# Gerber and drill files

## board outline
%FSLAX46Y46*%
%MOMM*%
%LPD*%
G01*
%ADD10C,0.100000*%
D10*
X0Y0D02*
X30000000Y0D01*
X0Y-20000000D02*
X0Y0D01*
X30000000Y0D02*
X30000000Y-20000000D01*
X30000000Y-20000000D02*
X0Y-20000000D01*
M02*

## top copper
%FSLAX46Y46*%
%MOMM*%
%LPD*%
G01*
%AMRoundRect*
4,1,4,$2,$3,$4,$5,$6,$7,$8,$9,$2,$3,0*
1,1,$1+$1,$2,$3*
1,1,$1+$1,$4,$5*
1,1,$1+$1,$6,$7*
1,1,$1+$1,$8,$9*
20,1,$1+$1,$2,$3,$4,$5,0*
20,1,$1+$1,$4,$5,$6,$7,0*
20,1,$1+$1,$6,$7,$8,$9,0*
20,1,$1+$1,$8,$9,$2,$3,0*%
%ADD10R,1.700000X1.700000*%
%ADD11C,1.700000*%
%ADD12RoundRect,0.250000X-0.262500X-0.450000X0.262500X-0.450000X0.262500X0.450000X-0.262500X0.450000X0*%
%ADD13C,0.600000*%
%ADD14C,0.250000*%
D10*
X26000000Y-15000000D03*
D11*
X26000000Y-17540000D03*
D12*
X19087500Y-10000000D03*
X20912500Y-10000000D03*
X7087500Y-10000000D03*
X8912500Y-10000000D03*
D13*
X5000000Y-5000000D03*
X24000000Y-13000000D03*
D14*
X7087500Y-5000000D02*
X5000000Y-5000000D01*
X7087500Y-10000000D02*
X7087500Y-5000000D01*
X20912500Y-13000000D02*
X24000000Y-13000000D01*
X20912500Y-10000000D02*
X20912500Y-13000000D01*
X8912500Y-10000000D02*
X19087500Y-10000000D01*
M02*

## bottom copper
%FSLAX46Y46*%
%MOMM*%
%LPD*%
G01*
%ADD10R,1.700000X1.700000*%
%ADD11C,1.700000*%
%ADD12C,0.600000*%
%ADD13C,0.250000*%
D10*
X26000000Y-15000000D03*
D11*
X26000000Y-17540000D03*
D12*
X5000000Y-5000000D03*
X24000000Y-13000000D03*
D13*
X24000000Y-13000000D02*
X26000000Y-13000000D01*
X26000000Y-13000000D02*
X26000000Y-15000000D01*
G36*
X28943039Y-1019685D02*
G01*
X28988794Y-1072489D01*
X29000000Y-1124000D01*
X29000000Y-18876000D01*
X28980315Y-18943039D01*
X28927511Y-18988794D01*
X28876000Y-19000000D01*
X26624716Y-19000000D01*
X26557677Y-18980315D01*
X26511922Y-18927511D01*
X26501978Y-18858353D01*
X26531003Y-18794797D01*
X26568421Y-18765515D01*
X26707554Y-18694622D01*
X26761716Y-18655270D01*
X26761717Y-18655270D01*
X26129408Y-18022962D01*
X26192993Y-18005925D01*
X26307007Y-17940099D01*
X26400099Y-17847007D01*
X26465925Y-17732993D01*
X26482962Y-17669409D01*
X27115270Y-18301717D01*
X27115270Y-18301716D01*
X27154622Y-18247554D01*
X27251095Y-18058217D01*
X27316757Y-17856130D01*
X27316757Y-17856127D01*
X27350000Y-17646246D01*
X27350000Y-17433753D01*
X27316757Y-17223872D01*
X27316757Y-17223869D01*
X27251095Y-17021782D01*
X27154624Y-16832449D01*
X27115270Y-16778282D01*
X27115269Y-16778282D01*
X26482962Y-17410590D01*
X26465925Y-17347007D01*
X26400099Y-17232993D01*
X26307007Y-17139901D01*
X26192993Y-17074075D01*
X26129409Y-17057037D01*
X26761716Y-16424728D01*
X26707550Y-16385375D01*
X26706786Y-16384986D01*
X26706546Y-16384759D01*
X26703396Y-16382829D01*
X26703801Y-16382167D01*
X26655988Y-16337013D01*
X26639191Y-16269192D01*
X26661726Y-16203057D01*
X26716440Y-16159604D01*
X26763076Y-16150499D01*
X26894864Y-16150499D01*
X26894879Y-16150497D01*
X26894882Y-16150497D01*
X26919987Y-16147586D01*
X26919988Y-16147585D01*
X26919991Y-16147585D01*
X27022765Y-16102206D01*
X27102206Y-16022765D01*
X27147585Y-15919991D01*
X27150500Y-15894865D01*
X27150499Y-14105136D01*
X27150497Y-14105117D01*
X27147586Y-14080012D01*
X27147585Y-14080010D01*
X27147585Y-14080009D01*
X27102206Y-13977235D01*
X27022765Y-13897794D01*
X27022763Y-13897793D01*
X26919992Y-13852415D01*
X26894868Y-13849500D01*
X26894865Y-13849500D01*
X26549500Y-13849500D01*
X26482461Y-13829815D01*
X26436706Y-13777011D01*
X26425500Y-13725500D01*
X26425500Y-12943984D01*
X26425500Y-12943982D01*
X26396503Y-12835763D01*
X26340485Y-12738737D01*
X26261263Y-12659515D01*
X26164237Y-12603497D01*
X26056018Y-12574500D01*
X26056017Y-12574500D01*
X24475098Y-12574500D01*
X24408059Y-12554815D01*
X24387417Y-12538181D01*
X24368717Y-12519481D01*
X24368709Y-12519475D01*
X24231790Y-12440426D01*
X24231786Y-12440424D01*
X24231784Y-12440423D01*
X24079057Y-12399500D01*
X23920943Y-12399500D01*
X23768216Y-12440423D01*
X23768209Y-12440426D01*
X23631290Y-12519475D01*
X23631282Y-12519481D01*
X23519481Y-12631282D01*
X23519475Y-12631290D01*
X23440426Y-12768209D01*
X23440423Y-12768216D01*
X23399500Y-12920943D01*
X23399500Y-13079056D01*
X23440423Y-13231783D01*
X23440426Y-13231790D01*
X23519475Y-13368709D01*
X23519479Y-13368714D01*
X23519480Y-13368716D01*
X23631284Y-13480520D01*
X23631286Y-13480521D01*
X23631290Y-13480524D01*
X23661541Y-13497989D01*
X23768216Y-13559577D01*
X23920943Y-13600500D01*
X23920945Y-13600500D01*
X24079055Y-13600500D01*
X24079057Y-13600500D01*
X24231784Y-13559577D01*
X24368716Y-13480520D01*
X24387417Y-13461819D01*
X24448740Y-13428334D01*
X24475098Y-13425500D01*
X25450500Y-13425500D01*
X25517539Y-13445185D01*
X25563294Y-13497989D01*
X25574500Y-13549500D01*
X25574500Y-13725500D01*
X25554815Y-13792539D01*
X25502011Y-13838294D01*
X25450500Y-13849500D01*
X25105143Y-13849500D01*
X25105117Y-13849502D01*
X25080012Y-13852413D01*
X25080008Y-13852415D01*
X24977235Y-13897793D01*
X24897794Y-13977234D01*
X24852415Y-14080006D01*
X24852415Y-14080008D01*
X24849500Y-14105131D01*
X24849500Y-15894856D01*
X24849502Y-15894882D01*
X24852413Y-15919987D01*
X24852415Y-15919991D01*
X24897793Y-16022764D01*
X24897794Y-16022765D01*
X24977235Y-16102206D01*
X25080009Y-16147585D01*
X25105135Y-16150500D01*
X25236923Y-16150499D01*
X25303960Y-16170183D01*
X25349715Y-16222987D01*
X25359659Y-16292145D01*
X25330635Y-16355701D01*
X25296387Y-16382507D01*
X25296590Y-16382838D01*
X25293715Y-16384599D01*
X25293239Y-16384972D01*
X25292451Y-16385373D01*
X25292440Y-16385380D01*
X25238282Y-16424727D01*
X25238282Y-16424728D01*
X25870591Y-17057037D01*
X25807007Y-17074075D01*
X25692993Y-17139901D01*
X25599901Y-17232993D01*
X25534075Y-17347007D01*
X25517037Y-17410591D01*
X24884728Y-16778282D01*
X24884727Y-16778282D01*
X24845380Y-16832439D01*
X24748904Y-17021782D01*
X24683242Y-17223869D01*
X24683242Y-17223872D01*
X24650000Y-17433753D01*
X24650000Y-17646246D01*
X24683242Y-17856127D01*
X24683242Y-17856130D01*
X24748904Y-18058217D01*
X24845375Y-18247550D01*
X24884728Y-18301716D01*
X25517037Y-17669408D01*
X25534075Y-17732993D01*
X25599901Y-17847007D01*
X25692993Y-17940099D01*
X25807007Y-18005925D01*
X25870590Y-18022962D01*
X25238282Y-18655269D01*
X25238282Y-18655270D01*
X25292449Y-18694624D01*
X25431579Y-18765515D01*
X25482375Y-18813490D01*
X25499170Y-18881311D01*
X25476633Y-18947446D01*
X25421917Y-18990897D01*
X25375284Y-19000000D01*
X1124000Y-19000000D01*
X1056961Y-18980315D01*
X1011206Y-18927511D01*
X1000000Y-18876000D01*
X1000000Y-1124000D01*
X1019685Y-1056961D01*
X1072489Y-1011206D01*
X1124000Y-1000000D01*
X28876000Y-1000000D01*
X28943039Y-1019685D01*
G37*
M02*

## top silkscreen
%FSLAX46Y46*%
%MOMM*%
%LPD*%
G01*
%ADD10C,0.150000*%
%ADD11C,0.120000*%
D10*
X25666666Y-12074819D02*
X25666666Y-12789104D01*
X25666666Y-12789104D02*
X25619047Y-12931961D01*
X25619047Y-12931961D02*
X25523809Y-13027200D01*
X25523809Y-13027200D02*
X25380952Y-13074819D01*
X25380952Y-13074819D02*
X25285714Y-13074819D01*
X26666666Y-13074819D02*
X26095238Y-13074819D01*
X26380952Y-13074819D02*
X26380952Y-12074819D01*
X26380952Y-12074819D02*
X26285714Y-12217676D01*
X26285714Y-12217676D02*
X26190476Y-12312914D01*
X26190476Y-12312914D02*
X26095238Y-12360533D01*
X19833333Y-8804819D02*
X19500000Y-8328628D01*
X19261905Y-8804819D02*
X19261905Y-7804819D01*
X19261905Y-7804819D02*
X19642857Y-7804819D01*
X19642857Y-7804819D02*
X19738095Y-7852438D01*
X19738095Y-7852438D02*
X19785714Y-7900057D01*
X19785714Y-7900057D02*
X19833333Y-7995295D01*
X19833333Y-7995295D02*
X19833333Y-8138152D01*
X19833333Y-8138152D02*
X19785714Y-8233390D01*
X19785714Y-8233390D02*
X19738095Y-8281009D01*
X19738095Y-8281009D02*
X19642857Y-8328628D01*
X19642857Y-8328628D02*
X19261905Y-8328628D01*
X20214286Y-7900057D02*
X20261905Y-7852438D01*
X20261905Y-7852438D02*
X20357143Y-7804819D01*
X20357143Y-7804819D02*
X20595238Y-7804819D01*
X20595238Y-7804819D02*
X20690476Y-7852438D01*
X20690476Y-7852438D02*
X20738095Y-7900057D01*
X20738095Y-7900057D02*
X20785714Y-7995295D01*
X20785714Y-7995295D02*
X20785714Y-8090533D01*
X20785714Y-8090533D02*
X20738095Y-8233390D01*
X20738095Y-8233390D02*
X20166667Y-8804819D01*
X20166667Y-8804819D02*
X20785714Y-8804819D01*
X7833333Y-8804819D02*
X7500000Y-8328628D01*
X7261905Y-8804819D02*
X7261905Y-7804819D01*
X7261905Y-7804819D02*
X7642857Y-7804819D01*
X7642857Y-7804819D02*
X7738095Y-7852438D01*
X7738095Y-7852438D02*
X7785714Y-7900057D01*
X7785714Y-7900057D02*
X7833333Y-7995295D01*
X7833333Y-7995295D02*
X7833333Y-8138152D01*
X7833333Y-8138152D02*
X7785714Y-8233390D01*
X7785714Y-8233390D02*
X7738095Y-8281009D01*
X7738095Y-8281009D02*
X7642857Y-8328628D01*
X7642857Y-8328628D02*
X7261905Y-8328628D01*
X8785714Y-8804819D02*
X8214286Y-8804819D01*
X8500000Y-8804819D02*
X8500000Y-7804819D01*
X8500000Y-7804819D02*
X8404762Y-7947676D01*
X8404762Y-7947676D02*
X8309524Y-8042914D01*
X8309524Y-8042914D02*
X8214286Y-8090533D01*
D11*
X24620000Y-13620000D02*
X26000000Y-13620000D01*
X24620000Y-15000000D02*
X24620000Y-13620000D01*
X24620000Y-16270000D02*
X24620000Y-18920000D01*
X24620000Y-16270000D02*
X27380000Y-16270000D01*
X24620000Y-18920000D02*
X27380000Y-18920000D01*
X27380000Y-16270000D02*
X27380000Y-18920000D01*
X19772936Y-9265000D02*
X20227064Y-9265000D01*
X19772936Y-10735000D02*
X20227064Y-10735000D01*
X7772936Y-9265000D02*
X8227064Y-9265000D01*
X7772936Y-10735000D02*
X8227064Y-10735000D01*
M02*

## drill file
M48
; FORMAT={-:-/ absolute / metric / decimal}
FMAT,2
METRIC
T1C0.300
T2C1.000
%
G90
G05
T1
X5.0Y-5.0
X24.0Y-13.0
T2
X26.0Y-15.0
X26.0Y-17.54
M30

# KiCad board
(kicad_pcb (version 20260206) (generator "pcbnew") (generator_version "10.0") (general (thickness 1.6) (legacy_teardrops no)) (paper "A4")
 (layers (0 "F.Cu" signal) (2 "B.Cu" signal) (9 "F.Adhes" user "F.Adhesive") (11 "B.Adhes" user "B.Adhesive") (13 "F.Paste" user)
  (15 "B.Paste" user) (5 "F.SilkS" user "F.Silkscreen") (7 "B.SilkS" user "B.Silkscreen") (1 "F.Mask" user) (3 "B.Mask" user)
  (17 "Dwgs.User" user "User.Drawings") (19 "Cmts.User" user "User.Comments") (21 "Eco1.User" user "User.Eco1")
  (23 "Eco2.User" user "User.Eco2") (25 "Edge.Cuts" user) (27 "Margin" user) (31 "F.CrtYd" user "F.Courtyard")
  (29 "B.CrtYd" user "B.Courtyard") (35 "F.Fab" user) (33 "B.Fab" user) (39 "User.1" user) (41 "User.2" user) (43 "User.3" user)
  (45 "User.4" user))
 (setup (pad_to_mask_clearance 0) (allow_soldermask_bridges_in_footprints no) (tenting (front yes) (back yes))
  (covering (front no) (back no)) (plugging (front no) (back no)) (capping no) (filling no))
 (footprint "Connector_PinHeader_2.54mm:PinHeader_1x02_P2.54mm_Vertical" (layer "F.Cu") (at 26 15)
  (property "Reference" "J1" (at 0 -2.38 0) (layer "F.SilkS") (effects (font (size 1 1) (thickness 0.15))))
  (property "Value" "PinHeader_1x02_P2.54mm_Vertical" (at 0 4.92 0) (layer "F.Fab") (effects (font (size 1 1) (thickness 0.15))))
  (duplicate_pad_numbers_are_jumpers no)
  (fp_line (start -1.38 -1.38) (end 0 -1.38) (stroke (width 0.12) (type solid)) (layer "F.SilkS"))
  (fp_line (start -1.38 0) (end -1.38 -1.38) (stroke (width 0.12) (type solid)) (layer "F.SilkS"))
  (fp_line (start -1.38 1.27) (end -1.38 3.92) (stroke (width 0.12) (type solid)) (layer "F.SilkS"))
  (fp_line (start -1.38 1.27) (end 1.38 1.27) (stroke (width 0.12) (type solid)) (layer "F.SilkS"))
  (fp_line (start -1.38 3.92) (end 1.38 3.92) (stroke (width 0.12) (type solid)) (layer "F.SilkS"))
  (fp_line (start 1.38 1.27) (end 1.38 3.92) (stroke (width 0.12) (type solid)) (layer "F.SilkS"))
  (pad "1" thru_hole rect (at 0 0) (size 1.7 1.7) (drill 1) (layers "*.Cu" "*.Mask") (remove_unused_layers no) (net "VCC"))
  (pad "2" thru_hole circle (at 0 2.54) (size 1.7 1.7) (drill 1) (layers "*.Cu" "*.Mask") (remove_unused_layers no) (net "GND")))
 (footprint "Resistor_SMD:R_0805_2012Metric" (layer "F.Cu") (at 20 10)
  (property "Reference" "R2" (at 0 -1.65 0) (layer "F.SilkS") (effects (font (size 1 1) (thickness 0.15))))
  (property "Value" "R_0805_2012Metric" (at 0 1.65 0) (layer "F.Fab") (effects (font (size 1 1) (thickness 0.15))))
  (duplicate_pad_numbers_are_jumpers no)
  (fp_line (start -0.227064 -0.735) (end 0.227064 -0.735) (stroke (width 0.12) (type solid)) (layer "F.SilkS"))
  (fp_line (start -0.227064 0.735) (end 0.227064 0.735) (stroke (width 0.12) (type solid)) (layer "F.SilkS"))
  (pad "1" smd roundrect (at -0.9125 0) (size 1.025 1.4) (layers "F.Cu" "F.Mask" "F.Paste") (roundrect_rratio 0.243902) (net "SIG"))
  (pad "2" smd roundrect (at 0.9125 0) (size 1.025 1.4) (layers "F.Cu" "F.Mask" "F.Paste") (roundrect_rratio 0.243902) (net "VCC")))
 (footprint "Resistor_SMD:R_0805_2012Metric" (layer "F.Cu") (at 8 10)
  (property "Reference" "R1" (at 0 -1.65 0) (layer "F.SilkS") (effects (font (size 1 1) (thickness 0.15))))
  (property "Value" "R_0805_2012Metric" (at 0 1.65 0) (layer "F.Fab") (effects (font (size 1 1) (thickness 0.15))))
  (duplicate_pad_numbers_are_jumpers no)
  (fp_line (start -0.227064 -0.735) (end 0.227064 -0.735) (stroke (width 0.12) (type solid)) (layer "F.SilkS"))
  (fp_line (start -0.227064 0.735) (end 0.227064 0.735) (stroke (width 0.12) (type solid)) (layer "F.SilkS"))
  (pad "1" smd roundrect (at -0.9125 0) (size 1.025 1.4) (layers "F.Cu" "F.Mask" "F.Paste") (roundrect_rratio 0.243902) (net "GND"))
  (pad "2" smd roundrect (at 0.9125 0) (size 1.025 1.4) (layers "F.Cu" "F.Mask" "F.Paste") (roundrect_rratio 0.243902) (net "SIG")))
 (gr_line (start 0 0) (end 30 0) (stroke (width 0.1) (type default)) (layer "Edge.Cuts"))
 (gr_line (start 0 20) (end 0 0) (stroke (width 0.1) (type default)) (layer "Edge.Cuts"))
 (gr_line (start 30 0) (end 30 20) (stroke (width 0.1) (type default)) (layer "Edge.Cuts"))
 (gr_line (start 30 20) (end 0 20) (stroke (width 0.1) (type default)) (layer "Edge.Cuts"))
 (segment (start 7.0875 5) (end 5 5) (width 0.25) (layer "F.Cu") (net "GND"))
 (segment (start 7.0875 10) (end 7.0875 5) (width 0.25) (layer "F.Cu") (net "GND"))
 (via (at 5 5) (size 0.6) (drill 0.3) (layers "F.Cu" "B.Cu") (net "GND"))
 (segment (start 20.9125 13) (end 24 13) (width 0.25) (layer "F.Cu") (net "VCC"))
 (segment (start 20.9125 10) (end 20.9125 13) (width 0.25) (layer "F.Cu") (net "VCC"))
 (via (at 24 13) (size 0.6) (drill 0.3) (layers "F.Cu" "B.Cu") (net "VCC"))
 (segment (start 24 13) (end 26 13) (width 0.25) (layer "B.Cu") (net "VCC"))
 (segment (start 26 13) (end 26 15) (width 0.25) (layer "B.Cu") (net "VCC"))
 (segment (start 8.9125 10) (end 19.0875 10) (width 0.25) (layer "F.Cu") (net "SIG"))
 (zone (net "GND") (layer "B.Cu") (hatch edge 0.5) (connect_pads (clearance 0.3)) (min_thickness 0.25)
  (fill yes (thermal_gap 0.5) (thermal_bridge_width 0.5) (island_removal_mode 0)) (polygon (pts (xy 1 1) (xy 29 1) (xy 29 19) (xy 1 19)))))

